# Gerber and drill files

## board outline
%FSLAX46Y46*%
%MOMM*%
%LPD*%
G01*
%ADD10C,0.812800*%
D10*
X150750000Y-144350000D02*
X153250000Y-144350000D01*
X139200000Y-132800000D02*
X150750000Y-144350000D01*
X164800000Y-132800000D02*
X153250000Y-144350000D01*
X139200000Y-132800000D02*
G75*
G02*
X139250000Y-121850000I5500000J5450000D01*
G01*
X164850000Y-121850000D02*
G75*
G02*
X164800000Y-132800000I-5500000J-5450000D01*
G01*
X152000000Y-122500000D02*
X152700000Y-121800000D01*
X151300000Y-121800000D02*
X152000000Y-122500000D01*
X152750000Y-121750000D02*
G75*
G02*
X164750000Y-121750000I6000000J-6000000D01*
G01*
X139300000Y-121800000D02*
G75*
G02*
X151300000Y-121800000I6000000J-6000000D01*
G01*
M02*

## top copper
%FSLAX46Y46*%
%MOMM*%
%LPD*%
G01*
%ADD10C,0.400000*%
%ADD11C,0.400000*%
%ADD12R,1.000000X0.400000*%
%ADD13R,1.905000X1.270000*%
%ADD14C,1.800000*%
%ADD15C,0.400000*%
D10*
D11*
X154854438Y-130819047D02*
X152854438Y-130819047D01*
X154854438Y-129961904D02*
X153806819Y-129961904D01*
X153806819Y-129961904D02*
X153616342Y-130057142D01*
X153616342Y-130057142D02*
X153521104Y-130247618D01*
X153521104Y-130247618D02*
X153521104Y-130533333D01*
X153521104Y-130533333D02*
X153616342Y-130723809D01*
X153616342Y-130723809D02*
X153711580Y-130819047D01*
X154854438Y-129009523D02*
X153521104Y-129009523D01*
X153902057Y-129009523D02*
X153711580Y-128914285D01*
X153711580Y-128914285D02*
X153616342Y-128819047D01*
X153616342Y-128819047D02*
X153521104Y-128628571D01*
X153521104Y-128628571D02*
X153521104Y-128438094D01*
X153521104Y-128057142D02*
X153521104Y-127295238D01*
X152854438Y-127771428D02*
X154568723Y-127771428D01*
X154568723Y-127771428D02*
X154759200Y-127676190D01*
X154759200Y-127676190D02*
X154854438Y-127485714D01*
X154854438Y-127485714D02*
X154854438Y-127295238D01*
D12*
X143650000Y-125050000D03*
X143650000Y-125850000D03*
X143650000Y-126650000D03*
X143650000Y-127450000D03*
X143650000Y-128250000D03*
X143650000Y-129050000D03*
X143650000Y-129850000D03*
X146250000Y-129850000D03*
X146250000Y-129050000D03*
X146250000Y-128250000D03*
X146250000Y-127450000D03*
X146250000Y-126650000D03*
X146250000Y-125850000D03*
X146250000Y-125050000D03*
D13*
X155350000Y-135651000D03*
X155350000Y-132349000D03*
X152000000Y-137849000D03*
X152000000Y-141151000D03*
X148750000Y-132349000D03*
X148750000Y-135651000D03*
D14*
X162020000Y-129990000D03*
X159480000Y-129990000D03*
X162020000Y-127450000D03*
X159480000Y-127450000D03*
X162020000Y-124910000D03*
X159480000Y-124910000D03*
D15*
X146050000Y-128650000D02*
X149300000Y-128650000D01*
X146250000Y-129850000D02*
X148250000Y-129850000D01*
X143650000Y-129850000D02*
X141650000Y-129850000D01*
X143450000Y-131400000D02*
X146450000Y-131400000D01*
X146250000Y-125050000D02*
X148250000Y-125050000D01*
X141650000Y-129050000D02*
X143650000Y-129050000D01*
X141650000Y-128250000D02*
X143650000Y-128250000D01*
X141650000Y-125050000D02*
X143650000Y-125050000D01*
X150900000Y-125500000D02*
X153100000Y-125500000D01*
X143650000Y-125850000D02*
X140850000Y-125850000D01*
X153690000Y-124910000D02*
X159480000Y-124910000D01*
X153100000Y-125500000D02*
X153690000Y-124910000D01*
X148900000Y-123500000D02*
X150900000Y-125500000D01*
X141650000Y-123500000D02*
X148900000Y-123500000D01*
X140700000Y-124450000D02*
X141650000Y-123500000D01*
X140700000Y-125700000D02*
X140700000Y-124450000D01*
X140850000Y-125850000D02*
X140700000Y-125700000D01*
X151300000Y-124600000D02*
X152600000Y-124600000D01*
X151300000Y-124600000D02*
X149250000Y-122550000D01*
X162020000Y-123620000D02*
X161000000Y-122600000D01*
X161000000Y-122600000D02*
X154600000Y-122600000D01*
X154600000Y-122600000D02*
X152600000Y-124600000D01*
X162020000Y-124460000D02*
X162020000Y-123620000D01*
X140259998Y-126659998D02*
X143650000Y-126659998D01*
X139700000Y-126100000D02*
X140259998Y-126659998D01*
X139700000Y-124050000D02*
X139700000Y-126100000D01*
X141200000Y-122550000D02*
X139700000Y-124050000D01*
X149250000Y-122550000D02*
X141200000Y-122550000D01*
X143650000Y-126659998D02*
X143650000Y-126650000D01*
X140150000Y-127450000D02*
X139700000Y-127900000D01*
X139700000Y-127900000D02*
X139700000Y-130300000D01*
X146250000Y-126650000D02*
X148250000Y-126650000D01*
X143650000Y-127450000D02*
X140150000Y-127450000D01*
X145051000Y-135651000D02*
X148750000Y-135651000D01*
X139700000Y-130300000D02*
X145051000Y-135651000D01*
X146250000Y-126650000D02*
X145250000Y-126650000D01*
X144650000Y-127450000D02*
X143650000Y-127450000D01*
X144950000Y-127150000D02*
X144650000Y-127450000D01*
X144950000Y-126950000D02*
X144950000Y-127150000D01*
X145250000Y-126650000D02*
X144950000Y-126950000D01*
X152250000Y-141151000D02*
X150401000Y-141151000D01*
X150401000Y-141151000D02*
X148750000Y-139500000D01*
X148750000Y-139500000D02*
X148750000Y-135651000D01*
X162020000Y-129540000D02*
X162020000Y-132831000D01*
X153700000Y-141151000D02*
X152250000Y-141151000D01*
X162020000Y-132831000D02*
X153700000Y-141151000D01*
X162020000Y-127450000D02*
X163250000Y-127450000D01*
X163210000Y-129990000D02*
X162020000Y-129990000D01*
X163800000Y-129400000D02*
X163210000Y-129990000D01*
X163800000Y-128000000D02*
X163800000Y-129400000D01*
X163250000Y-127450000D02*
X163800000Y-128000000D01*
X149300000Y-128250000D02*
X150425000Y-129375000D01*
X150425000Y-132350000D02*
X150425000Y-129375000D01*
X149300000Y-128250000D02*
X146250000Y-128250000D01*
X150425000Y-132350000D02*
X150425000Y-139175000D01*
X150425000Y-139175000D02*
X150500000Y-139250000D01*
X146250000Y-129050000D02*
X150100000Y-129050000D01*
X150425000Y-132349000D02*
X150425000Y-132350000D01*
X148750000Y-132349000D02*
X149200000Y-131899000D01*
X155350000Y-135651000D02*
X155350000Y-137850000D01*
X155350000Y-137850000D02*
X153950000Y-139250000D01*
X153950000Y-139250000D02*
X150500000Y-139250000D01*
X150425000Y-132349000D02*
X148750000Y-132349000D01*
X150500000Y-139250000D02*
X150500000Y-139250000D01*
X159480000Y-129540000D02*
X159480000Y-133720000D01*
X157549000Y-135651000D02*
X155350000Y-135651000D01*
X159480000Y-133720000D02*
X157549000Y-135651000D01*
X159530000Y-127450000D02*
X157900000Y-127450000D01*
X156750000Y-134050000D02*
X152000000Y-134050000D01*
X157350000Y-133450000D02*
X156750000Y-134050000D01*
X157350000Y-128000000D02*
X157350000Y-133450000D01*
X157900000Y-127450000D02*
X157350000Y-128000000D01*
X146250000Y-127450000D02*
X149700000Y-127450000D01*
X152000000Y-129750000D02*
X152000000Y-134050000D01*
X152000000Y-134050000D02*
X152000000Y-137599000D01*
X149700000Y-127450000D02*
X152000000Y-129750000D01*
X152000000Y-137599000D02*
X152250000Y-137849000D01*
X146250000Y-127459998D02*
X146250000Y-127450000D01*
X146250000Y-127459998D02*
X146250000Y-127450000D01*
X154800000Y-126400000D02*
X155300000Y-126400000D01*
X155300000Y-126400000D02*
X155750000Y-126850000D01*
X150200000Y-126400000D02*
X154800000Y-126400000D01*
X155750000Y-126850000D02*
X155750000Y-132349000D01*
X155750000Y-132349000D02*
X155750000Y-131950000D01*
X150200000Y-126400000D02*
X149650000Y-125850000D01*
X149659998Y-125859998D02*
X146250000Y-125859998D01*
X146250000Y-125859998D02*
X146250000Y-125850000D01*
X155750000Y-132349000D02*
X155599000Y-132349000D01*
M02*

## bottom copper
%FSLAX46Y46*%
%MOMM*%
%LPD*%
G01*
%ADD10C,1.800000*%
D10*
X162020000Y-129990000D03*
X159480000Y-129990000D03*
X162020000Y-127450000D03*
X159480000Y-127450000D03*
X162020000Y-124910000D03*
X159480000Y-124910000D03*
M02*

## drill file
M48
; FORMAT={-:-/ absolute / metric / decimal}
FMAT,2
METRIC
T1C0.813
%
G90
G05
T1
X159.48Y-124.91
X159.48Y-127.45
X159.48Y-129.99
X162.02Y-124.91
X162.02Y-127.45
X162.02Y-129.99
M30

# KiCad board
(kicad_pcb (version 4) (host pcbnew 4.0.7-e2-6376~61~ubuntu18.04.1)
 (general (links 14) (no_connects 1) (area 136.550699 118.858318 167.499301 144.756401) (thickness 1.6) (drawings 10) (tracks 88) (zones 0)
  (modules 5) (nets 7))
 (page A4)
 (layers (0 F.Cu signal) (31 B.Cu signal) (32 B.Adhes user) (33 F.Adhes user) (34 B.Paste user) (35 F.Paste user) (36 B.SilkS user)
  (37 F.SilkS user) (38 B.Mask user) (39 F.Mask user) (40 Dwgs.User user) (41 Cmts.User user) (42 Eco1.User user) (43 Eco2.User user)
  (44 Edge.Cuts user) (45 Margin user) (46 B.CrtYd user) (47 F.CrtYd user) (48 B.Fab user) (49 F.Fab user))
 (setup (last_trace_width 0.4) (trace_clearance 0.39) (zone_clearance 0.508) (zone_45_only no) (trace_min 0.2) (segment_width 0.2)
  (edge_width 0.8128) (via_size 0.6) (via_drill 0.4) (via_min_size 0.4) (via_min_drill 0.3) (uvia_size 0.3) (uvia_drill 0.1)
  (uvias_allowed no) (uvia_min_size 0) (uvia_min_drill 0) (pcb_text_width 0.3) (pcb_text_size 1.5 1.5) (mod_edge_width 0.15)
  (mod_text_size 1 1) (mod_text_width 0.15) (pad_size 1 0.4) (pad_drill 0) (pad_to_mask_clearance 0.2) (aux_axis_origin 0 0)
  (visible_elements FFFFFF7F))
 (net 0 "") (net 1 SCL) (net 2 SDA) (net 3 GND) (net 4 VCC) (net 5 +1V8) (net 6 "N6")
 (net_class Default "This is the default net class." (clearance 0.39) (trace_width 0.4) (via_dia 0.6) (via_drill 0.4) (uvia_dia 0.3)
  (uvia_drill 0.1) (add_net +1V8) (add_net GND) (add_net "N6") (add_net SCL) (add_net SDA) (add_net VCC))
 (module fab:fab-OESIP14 (layer F.Cu) (at 144.95 127.45)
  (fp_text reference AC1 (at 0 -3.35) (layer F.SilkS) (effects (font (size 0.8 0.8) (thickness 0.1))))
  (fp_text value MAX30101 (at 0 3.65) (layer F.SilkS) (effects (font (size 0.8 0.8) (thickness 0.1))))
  (pad 1 smd rect (at -1.3 -2.4) (size 1 0.4) (layers F.Cu F.Paste F.Mask))
  (pad 2 smd rect (at -1.3 -1.6) (size 1 0.4) (layers F.Cu F.Paste F.Mask) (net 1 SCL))
  (pad 3 smd rect (at -1.3 -0.8) (size 1 0.4) (layers F.Cu F.Paste F.Mask) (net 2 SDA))
  (pad 4 smd rect (at -1.3 0) (size 1 0.4) (layers F.Cu F.Paste F.Mask) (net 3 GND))
  (pad 5 smd rect (at -1.3 0.8) (size 1 0.4) (layers F.Cu F.Paste F.Mask))
  (pad 6 smd rect (at -1.3 1.6) (size 1 0.4) (layers F.Cu F.Paste F.Mask))
  (pad 7 smd rect (at -1.3 2.4) (size 1 0.4) (layers F.Cu F.Paste F.Mask))
  (pad 8 smd rect (at 1.3 2.4) (size 1 0.4) (layers F.Cu F.Paste F.Mask))
  (pad 9 smd rect (at 1.3 1.6) (size 1 0.4) (layers F.Cu F.Paste F.Mask) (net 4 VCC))
  (pad 10 smd rect (at 1.3 0.8) (size 1 0.4) (layers F.Cu F.Paste F.Mask) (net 4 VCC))
  (pad 11 smd rect (at 1.3 0) (size 1 0.4) (layers F.Cu F.Paste F.Mask) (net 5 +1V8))
  (pad 12 smd rect (at 1.3 -0.8) (size 1 0.4) (layers F.Cu F.Paste F.Mask) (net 3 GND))
  (pad 13 smd rect (at 1.3 -1.6) (size 1 0.4) (layers F.Cu F.Paste F.Mask) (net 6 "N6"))
  (pad 14 smd rect (at 1.3 -2.4) (size 1 0.4) (layers F.Cu F.Paste F.Mask)))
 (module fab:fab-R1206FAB (layer F.Cu) (at 155.35 134 90)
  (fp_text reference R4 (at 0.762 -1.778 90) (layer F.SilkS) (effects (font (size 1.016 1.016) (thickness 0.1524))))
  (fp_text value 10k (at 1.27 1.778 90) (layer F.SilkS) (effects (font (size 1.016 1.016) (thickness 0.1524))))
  (pad 1 smd rect (at -1.651 0 90) (size 1.27 1.905) (layers F.Cu F.Paste F.Mask) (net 4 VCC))
  (pad 2 smd rect (at 1.651 0 90) (size 1.27 1.905) (layers F.Cu F.Paste F.Mask) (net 6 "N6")))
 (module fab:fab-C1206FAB (layer F.Cu) (at 152 139.5 270)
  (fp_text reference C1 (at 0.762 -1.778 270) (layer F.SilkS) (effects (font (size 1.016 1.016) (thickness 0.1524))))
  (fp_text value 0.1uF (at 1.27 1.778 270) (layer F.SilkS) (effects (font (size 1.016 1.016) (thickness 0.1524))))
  (pad 1 smd rect (at -1.651 0 270) (size 1.27 1.905) (layers F.Cu F.Paste F.Mask) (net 5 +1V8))
  (pad 2 smd rect (at 1.651 0 270) (size 1.27 1.905) (layers F.Cu F.Paste F.Mask) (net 3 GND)))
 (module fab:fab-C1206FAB (layer F.Cu) (at 148.75 134 270)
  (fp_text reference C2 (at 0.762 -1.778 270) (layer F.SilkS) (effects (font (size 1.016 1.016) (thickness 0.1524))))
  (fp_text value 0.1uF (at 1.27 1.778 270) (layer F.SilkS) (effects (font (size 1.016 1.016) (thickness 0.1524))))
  (pad 1 smd rect (at -1.651 0 270) (size 1.27 1.905) (layers F.Cu F.Paste F.Mask) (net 4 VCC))
  (pad 2 smd rect (at 1.651 0 270) (size 1.27 1.905) (layers F.Cu F.Paste F.Mask) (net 3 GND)))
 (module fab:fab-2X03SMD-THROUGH (layer F.Cu) (at 160.75 127.45 180)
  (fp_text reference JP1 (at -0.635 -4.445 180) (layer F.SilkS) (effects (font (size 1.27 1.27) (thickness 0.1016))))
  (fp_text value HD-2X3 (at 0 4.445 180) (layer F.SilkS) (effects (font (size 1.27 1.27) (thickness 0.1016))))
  (pad 1 thru_hole circle (at -1.27 -2.54 180) (size 1.8 1.8) (drill 0.8128) (layers F.Cu F.Paste F.Mask) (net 3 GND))
  (pad 2 thru_hole circle (at 1.27 -2.54 180) (size 1.8 1.8) (drill 0.8128) (layers F.Cu F.Paste F.Mask) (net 4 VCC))
  (pad 3 thru_hole circle (at -1.27 0 180) (size 1.8 1.8) (drill 0.8128) (layers F.Cu F.Paste F.Mask) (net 3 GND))
  (pad 4 thru_hole circle (at 1.27 0 180) (size 1.8 1.8) (drill 0.8128) (layers F.Cu F.Paste F.Mask) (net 5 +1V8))
  (pad 5 thru_hole circle (at -1.27 2.54 180) (size 1.8 1.8) (drill 0.8128) (layers F.Cu B.Paste F.Mask) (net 2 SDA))
  (pad 6 thru_hole circle (at 1.27 2.54 180) (size 1.8 1.8) (drill 0.8128) (layers F.Cu F.Paste F.Mask) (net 1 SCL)))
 (gr_line (start 150.75 144.35) (end 153.25 144.35) (angle 90) (layer Edge.Cuts) (width 0.8128))
 (gr_line (start 139.2 132.8) (end 150.75 144.35) (angle 90) (layer Edge.Cuts) (width 0.8128))
 (gr_line (start 164.8 132.8) (end 153.25 144.35) (angle 90) (layer Edge.Cuts) (width 0.8128))
 (gr_arc (start 144.7 127.35) (end 139.2 132.8) (angle 90) (layer Edge.Cuts) (width 0.8128))
 (gr_arc (start 159.35 127.3) (end 164.85 121.85) (angle 90) (layer Edge.Cuts) (width 0.8128))
 (gr_line (start 152 122.5) (end 152.7 121.8) (angle 90) (layer Edge.Cuts) (width 0.8128))
 (gr_line (start 151.3 121.8) (end 152 122.5) (angle 90) (layer Edge.Cuts) (width 0.8128))
 (gr_arc (start 158.75 127.75) (end 152.75 121.75) (angle 90) (layer Edge.Cuts) (width 0.8128))
 (gr_arc (start 145.3 127.8) (end 139.3 121.8) (angle 90) (layer Edge.Cuts) (width 0.8128))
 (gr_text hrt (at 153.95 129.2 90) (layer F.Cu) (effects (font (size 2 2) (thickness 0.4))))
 (segment (start 146.05 128.65) (end 149.3 128.65) (width 0.4) (layer F.Cu) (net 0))
 (segment (start 146.25 129.85) (end 148.25 129.85) (width 0.4) (layer F.Cu) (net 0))
 (segment (start 143.65 129.85) (end 141.65 129.85) (width 0.4) (layer F.Cu) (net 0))
 (segment (start 143.45 131.4) (end 146.45 131.4) (width 0.4) (layer F.Cu) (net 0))
 (segment (start 146.25 125.05) (end 148.25 125.05) (width 0.4) (layer F.Cu) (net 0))
 (segment (start 141.65 129.05) (end 143.65 129.05) (width 0.4) (layer F.Cu) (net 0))
 (segment (start 141.65 128.25) (end 143.65 128.25) (width 0.4) (layer F.Cu) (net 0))
 (segment (start 141.65 125.05) (end 143.65 125.05) (width 0.4) (layer F.Cu) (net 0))
 (segment (start 150.9 125.5) (end 153.1 125.5) (width 0.4) (layer F.Cu) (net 1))
 (segment (start 143.65 125.85) (end 140.85 125.85) (width 0.4) (layer F.Cu) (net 1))
 (segment (start 153.69 124.91) (end 159.48 124.91) (width 0.4) (layer F.Cu) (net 1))
 (segment (start 153.1 125.5) (end 153.69 124.91) (width 0.4) (layer F.Cu) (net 1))
 (segment (start 148.9 123.5) (end 150.9 125.5) (width 0.4) (layer F.Cu) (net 1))
 (segment (start 141.65 123.5) (end 148.9 123.5) (width 0.4) (layer F.Cu) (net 1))
 (segment (start 140.7 124.45) (end 141.65 123.5) (width 0.4) (layer F.Cu) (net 1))
 (segment (start 140.7 125.7) (end 140.7 124.45) (width 0.4) (layer F.Cu) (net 1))
 (segment (start 140.85 125.85) (end 140.7 125.7) (width 0.4) (layer F.Cu) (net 1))
 (segment (start 151.3 124.6) (end 152.6 124.6) (width 0.4) (layer F.Cu) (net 2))
 (segment (start 151.3 124.6) (end 149.25 122.55) (width 0.4) (layer F.Cu) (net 2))
 (segment (start 162.02 123.62) (end 161 122.6) (width 0.4) (layer F.Cu) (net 2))
 (segment (start 161 122.6) (end 154.6 122.6) (width 0.4) (layer F.Cu) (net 2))
 (segment (start 154.6 122.6) (end 152.6 124.6) (width 0.4) (layer F.Cu) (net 2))
 (segment (start 162.02 124.46) (end 162.02 123.62) (width 0.4) (layer F.Cu) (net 2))
 (segment (start 140.259998 126.659998) (end 143.65 126.659998) (width 0.4) (layer F.Cu) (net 2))
 (segment (start 139.7 126.1) (end 140.259998 126.659998) (width 0.4) (layer F.Cu) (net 2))
 (segment (start 139.7 124.05) (end 139.7 126.1) (width 0.4) (layer F.Cu) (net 2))
 (segment (start 141.2 122.55) (end 139.7 124.05) (width 0.4) (layer F.Cu) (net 2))
 (segment (start 149.25 122.55) (end 141.2 122.55) (width 0.4) (layer F.Cu) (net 2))
 (segment (start 143.65 126.659998) (end 143.65 126.65) (width 0.4) (layer F.Cu) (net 2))
 (segment (start 140.15 127.45) (end 139.7 127.9) (width 0.4) (layer F.Cu) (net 3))
 (segment (start 139.7 127.9) (end 139.7 130.3) (width 0.4) (layer F.Cu) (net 3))
 (segment (start 146.25 126.65) (end 148.25 126.65) (width 0.4) (layer F.Cu) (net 3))
 (segment (start 143.65 127.45) (end 140.15 127.45) (width 0.4) (layer F.Cu) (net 3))
 (segment (start 145.051 135.651) (end 148.75 135.651) (width 0.4) (layer F.Cu) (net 3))
 (segment (start 139.7 130.3) (end 145.051 135.651) (width 0.4) (layer F.Cu) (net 3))
 (segment (start 146.25 126.65) (end 145.25 126.65) (width 0.4) (layer F.Cu) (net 3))
 (segment (start 144.65 127.45) (end 143.65 127.45) (width 0.4) (layer F.Cu) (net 3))
 (segment (start 144.95 127.15) (end 144.65 127.45) (width 0.4) (layer F.Cu) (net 3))
 (segment (start 144.95 126.95) (end 144.95 127.15) (width 0.4) (layer F.Cu) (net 3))
 (segment (start 145.25 126.65) (end 144.95 126.95) (width 0.4) (layer F.Cu) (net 3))
 (segment (start 152.25 141.151) (end 150.401 141.151) (width 0.4) (layer F.Cu) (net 3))
 (segment (start 150.401 141.151) (end 148.75 139.5) (width 0.4) (layer F.Cu) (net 3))
 (segment (start 148.75 139.5) (end 148.75 135.651) (width 0.4) (layer F.Cu) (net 3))
 (segment (start 162.02 129.54) (end 162.02 132.831) (width 0.4) (layer F.Cu) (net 3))
 (segment (start 153.7 141.151) (end 152.25 141.151) (width 0.4) (layer F.Cu) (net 3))
 (segment (start 162.02 132.831) (end 153.7 141.151) (width 0.4) (layer F.Cu) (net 3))
 (segment (start 162.02 127.45) (end 163.25 127.45) (width 0.4) (layer F.Cu) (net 3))
 (segment (start 163.21 129.99) (end 162.02 129.99) (width 0.4) (layer F.Cu) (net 3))
 (segment (start 163.8 129.4) (end 163.21 129.99) (width 0.4) (layer F.Cu) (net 3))
 (segment (start 163.8 128) (end 163.8 129.4) (width 0.4) (layer F.Cu) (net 3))
 (segment (start 163.25 127.45) (end 163.8 128) (width 0.4) (layer F.Cu) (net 3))
 (segment (start 149.3 128.25) (end 150.425 129.375) (width 0.4) (layer F.Cu) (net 4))
 (segment (start 150.425 132.35) (end 150.425 129.375) (width 0.4) (layer F.Cu) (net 4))
 (segment (start 149.3 128.25) (end 146.25 128.25) (width 0.4) (layer F.Cu) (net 4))
 (segment (start 150.425 132.35) (end 150.425 139.175) (width 0.4) (layer F.Cu) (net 4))
 (segment (start 150.425 139.175) (end 150.5 139.25) (width 0.4) (layer F.Cu) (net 4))
 (segment (start 146.25 129.05) (end 150.1 129.05) (width 0.4) (layer F.Cu) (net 4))
 (segment (start 150.425 132.349) (end 150.425 132.35) (width 0.4) (layer F.Cu) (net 4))
 (segment (start 148.75 132.349) (end 149.2 131.899) (width 0.4) (layer F.Cu) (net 4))
 (segment (start 155.35 135.651) (end 155.35 137.85) (width 0.4) (layer F.Cu) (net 4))
 (segment (start 155.35 137.85) (end 153.95 139.25) (width 0.4) (layer F.Cu) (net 4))
 (segment (start 153.95 139.25) (end 150.5 139.25) (width 0.4) (layer F.Cu) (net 4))
 (segment (start 150.425 132.349) (end 148.75 132.349) (width 0.4) (layer F.Cu) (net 4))
 (segment (start 150.5 139.25) (end 150.5 139.25) (width 0.4) (layer F.Cu) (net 4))
 (segment (start 159.48 129.54) (end 159.48 133.72) (width 0.4) (layer F.Cu) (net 4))
 (segment (start 157.549 135.651) (end 155.35 135.651) (width 0.4) (layer F.Cu) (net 4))
 (segment (start 159.48 133.72) (end 157.549 135.651) (width 0.4) (layer F.Cu) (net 4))
 (segment (start 159.53 127.45) (end 157.9 127.45) (width 0.4) (layer F.Cu) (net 5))
 (segment (start 156.75 134.05) (end 152 134.05) (width 0.4) (layer F.Cu) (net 5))
 (segment (start 157.35 133.45) (end 156.75 134.05) (width 0.4) (layer F.Cu) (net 5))
 (segment (start 157.35 128) (end 157.35 133.45) (width 0.4) (layer F.Cu) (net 5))
 (segment (start 157.9 127.45) (end 157.35 128) (width 0.4) (layer F.Cu) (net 5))
 (segment (start 146.25 127.45) (end 149.7 127.45) (width 0.4) (layer F.Cu) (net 5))
 (segment (start 152 129.75) (end 152 134.05) (width 0.4) (layer F.Cu) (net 5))
 (segment (start 152 134.05) (end 152 137.599) (width 0.4) (layer F.Cu) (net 5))
 (segment (start 149.7 127.45) (end 152 129.75) (width 0.4) (layer F.Cu) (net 5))
 (segment (start 152 137.599) (end 152.25 137.849) (width 0.4) (layer F.Cu) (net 5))
 (segment (start 146.25 127.459998) (end 146.25 127.45) (width 0.4) (layer F.Cu) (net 5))
 (segment (start 146.25 127.459998) (end 146.25 127.45) (width 0.4) (layer F.Cu) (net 5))
 (segment (start 154.8 126.4) (end 155.3 126.4) (width 0.4) (layer F.Cu) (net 6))
 (segment (start 155.3 126.4) (end 155.75 126.85) (width 0.4) (layer F.Cu) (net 6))
 (segment (start 150.2 126.4) (end 154.8 126.4) (width 0.4) (layer F.Cu) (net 6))
 (segment (start 155.75 126.85) (end 155.75 132.349) (width 0.4) (layer F.Cu) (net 6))
 (segment (start 155.75 132.349) (end 155.75 131.95) (width 0.4) (layer F.Cu) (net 6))
 (segment (start 150.2 126.4) (end 149.65 125.85) (width 0.4) (layer F.Cu) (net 6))
 (segment (start 149.659998 125.859998) (end 146.25 125.859998) (width 0.4) (layer F.Cu) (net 6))
 (segment (start 146.25 125.859998) (end 146.25 125.85) (width 0.4) (layer F.Cu) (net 6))
 (segment (start 155.75 132.349) (end 155.599 132.349) (width 0.4) (layer F.Cu) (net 6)))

